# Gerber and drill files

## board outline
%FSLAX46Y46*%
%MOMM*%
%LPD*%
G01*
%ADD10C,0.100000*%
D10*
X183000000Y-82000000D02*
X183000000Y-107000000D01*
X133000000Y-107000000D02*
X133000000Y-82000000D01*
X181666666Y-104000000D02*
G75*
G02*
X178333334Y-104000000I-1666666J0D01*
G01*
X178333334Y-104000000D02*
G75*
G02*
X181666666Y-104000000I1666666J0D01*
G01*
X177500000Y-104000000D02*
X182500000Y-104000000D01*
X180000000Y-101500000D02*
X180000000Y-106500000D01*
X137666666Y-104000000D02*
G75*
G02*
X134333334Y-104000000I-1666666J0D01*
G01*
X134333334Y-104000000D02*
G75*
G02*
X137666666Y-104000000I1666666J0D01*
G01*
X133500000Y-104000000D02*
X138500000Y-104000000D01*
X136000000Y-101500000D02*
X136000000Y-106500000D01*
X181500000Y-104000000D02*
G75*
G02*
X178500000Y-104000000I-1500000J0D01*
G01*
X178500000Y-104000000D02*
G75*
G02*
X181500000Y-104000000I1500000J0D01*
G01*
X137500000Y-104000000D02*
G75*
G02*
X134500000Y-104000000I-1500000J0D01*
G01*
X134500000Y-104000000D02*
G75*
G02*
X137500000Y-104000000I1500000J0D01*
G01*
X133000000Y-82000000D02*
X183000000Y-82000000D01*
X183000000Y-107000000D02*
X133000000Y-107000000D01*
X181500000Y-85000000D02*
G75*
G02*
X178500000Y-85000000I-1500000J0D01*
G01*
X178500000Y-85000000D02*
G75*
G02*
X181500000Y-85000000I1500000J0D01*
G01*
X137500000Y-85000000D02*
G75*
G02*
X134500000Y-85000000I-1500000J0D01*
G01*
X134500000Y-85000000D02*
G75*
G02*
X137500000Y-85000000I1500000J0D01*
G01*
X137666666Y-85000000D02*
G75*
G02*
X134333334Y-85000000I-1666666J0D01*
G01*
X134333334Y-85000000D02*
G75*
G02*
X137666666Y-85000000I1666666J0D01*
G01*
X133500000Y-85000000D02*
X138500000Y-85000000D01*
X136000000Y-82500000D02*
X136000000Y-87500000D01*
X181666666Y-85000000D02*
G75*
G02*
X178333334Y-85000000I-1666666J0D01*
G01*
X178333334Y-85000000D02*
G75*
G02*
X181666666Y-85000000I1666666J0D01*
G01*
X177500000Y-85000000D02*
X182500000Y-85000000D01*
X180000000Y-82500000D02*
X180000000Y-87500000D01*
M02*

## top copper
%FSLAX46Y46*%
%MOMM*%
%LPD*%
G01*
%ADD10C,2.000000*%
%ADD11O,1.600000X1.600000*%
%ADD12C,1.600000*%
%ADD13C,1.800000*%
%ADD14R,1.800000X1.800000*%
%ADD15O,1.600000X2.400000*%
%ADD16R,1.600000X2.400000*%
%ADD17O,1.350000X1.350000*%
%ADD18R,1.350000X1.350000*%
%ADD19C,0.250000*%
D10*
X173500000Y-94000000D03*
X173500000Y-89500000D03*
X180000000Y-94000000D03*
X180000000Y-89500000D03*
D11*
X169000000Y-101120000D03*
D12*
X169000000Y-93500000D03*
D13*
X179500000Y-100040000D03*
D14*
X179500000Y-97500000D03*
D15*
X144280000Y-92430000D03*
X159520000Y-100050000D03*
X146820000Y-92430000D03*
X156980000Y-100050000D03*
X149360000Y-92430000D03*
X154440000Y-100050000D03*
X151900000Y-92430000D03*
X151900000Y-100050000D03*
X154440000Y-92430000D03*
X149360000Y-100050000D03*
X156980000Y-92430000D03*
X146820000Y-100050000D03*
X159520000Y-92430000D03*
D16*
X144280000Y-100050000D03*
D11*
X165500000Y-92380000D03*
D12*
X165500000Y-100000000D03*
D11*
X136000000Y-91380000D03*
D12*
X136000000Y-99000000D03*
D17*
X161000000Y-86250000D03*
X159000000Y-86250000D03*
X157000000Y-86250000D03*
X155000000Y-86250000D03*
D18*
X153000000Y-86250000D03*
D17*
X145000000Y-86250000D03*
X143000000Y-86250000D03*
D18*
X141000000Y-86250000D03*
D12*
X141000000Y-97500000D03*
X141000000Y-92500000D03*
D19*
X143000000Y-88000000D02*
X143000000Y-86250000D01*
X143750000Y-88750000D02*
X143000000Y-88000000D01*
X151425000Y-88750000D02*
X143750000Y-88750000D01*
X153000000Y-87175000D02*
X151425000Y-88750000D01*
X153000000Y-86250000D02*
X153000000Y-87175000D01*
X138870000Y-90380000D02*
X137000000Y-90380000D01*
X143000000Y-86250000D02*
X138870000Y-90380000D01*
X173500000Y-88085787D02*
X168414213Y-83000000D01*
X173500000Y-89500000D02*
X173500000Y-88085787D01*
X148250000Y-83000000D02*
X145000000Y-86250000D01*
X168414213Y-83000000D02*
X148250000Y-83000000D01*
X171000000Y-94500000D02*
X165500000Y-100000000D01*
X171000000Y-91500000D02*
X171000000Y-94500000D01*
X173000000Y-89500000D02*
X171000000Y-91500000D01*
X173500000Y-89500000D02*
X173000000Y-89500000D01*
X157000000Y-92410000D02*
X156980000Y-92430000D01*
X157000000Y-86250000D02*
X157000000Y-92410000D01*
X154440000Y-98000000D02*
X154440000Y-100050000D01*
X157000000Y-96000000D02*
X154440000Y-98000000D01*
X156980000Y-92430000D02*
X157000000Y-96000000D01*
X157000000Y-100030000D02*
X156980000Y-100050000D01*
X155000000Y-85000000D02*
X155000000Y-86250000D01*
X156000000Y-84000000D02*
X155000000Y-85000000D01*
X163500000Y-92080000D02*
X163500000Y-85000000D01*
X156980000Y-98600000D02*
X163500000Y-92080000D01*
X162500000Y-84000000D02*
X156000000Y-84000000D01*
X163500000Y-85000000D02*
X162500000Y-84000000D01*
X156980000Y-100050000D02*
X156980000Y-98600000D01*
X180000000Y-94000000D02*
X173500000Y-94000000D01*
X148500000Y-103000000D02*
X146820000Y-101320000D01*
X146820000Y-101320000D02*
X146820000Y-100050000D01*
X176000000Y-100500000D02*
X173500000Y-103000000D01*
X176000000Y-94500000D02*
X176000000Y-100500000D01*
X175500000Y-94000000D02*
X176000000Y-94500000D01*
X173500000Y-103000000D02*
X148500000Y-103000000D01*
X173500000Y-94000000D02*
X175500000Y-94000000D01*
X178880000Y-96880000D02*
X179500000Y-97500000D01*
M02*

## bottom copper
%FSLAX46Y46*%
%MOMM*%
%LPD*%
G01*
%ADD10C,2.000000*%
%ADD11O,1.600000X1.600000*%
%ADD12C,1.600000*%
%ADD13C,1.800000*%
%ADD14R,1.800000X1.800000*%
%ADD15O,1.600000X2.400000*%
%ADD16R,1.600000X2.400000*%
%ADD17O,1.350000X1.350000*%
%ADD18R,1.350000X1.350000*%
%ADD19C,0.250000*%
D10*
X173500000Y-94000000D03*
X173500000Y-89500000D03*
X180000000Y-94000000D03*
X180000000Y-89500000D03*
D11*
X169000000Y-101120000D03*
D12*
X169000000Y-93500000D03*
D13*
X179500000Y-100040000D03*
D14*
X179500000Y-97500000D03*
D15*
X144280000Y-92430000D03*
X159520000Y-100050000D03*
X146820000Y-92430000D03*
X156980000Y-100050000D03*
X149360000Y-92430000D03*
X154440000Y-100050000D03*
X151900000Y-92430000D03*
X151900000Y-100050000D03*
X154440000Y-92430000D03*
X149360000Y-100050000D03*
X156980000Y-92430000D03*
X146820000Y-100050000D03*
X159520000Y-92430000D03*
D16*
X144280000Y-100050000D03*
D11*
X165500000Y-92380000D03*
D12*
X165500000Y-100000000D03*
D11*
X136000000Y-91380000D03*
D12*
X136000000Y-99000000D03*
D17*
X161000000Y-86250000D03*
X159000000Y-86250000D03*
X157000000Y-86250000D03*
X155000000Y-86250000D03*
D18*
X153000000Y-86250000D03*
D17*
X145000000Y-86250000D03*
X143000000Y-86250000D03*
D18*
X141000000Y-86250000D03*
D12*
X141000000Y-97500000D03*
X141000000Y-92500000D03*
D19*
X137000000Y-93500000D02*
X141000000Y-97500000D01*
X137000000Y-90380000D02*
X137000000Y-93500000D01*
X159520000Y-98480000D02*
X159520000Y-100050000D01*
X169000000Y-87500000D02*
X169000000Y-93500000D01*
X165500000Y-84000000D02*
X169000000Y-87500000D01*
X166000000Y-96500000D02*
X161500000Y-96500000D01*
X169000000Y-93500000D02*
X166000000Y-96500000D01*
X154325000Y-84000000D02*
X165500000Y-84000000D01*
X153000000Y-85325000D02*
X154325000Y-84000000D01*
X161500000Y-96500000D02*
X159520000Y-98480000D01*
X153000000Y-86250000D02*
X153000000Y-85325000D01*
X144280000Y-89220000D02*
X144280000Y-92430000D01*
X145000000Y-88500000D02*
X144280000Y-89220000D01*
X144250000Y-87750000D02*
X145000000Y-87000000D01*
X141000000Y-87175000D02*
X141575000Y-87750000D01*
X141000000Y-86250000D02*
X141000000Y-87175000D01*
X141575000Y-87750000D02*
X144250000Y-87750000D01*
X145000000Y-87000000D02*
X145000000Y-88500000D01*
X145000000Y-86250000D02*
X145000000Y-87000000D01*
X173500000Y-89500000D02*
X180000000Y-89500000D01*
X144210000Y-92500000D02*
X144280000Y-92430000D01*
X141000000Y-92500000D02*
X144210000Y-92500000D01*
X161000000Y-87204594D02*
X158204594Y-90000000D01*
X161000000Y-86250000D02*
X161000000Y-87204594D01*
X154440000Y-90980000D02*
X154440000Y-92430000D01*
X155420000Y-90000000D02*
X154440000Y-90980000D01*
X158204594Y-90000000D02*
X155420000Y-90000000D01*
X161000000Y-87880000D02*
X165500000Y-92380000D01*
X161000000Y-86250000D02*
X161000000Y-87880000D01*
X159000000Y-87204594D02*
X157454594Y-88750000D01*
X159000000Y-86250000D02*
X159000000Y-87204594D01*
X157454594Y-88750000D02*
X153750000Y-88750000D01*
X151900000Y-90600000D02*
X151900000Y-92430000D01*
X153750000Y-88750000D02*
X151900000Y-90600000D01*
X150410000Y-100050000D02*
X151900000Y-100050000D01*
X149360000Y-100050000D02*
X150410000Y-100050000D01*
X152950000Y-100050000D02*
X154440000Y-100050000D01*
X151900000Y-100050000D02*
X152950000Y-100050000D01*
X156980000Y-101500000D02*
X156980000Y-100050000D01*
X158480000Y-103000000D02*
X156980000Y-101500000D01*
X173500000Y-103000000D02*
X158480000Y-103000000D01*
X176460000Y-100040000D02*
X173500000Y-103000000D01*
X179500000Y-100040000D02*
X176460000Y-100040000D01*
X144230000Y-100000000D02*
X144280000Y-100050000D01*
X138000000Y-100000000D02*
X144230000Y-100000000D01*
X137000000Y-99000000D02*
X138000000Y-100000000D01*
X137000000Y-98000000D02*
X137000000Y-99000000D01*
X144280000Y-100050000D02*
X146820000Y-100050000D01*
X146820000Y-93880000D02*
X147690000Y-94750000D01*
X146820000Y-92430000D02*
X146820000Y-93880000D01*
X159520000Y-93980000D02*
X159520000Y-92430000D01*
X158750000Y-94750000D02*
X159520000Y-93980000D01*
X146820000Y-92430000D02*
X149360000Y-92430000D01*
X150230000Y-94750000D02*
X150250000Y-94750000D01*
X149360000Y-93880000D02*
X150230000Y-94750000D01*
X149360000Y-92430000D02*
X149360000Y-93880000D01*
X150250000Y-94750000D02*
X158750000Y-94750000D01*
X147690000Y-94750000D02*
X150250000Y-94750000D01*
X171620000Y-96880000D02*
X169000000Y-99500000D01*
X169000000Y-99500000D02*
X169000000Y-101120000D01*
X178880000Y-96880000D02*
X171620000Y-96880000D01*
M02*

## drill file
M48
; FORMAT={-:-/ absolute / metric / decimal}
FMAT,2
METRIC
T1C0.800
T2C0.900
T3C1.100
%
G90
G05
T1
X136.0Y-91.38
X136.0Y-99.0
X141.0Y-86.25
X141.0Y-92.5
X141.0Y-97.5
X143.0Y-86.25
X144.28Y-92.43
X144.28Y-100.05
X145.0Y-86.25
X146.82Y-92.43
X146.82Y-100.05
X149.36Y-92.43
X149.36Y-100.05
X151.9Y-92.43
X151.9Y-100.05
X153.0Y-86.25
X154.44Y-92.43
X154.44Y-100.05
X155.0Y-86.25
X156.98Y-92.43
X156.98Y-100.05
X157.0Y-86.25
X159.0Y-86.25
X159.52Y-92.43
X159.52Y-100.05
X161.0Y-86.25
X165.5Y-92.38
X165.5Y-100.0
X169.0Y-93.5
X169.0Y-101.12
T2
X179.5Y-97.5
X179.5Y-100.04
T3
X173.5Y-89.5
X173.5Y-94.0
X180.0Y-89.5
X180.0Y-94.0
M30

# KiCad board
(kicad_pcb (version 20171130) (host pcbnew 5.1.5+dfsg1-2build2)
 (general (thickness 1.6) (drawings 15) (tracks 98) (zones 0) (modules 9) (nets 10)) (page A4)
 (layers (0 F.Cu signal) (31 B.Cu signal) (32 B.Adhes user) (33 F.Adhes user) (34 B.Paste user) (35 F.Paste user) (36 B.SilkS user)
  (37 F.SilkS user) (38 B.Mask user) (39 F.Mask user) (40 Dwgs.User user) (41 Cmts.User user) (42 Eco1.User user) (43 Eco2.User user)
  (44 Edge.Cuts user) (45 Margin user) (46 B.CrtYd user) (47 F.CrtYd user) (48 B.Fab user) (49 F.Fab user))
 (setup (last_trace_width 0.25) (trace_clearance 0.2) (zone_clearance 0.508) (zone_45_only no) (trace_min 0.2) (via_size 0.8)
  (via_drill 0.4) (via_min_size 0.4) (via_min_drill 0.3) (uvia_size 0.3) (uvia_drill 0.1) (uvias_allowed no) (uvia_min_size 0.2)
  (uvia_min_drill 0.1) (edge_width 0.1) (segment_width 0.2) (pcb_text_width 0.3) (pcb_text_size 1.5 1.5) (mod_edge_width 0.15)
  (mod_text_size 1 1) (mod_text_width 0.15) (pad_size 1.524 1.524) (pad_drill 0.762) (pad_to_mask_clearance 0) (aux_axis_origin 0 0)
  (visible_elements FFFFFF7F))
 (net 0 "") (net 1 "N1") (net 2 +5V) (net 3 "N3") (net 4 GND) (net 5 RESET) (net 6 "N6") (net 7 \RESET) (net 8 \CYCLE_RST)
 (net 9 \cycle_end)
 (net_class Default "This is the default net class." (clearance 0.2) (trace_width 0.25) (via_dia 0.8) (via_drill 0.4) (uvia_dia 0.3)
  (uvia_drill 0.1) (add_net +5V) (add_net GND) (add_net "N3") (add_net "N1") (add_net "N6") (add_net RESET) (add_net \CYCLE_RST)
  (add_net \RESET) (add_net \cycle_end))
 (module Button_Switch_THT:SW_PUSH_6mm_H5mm (layer F.Cu) (at 180 94 180)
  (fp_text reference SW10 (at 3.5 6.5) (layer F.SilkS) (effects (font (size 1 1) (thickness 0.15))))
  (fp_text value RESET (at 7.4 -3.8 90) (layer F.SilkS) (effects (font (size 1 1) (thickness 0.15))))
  (pad 1 thru_hole circle (at 6.5 0 270) (size 2 2) (drill 1.1) (layers *.Cu *.Mask) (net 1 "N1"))
  (pad 2 thru_hole circle (at 6.5 4.5 270) (size 2 2) (drill 1.1) (layers *.Cu *.Mask) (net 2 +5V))
  (pad 1 thru_hole circle (at 0 0 270) (size 2 2) (drill 1.1) (layers *.Cu *.Mask) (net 1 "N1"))
  (pad 2 thru_hole circle (at 0 4.5 270) (size 2 2) (drill 1.1) (layers *.Cu *.Mask) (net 2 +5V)))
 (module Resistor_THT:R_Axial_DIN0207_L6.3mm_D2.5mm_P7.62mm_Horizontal (layer F.Cu) (at 169 93.5 270)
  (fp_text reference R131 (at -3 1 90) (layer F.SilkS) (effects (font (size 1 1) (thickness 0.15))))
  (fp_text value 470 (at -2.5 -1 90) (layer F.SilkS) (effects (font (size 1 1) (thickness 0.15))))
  (pad 2 thru_hole oval (at 7.62 0 270) (size 1.6 1.6) (drill 0.8) (layers *.Cu *.Mask) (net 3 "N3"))
  (pad 1 thru_hole circle (at 0 0 270) (size 1.6 1.6) (drill 0.8) (layers *.Cu *.Mask) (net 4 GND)))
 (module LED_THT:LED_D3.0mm (layer F.Cu) (at 179.5 97.5 270)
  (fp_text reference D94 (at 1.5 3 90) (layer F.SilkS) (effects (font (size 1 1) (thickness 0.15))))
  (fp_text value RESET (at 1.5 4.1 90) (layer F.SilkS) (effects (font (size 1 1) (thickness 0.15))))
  (pad 2 thru_hole circle (at 2.54 0 270) (size 1.8 1.8) (drill 0.9) (layers *.Cu *.Mask) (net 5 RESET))
  (pad 1 thru_hole rect (at 0 0 270) (size 1.8 1.8) (drill 0.9) (layers *.Cu *.Mask) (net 3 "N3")))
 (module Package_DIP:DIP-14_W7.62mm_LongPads (layer F.Cu) (at 144.28 100.05 90)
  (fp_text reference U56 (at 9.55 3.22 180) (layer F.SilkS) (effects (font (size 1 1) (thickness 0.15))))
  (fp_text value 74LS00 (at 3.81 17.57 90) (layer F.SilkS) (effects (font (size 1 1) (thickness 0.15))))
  (pad 14 thru_hole oval (at 7.62 0 90) (size 2.4 1.6) (drill 0.8) (layers *.Cu *.Mask) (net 2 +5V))
  (pad 7 thru_hole oval (at 0 15.24 90) (size 2.4 1.6) (drill 0.8) (layers *.Cu *.Mask) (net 4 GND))
  (pad 13 thru_hole oval (at 7.62 2.54 90) (size 2.4 1.6) (drill 0.8) (layers *.Cu *.Mask) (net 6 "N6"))
  (pad 6 thru_hole oval (at 0 12.7 90) (size 2.4 1.6) (drill 0.8) (layers *.Cu *.Mask) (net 5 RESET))
  (pad 12 thru_hole oval (at 7.62 5.08 90) (size 2.4 1.6) (drill 0.8) (layers *.Cu *.Mask) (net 6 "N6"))
  (pad 5 thru_hole oval (at 0 10.16 90) (size 2.4 1.6) (drill 0.8) (layers *.Cu *.Mask) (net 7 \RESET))
  (pad 11 thru_hole oval (at 7.62 7.62 90) (size 2.4 1.6) (drill 0.8) (layers *.Cu *.Mask) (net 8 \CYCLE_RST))
  (pad 4 thru_hole oval (at 0 7.62 90) (size 2.4 1.6) (drill 0.8) (layers *.Cu *.Mask) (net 7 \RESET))
  (pad 10 thru_hole oval (at 7.62 10.16 90) (size 2.4 1.6) (drill 0.8) (layers *.Cu *.Mask) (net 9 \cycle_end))
  (pad 3 thru_hole oval (at 0 5.08 90) (size 2.4 1.6) (drill 0.8) (layers *.Cu *.Mask) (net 7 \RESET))
  (pad 9 thru_hole oval (at 7.62 12.7 90) (size 2.4 1.6) (drill 0.8) (layers *.Cu *.Mask) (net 7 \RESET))
  (pad 2 thru_hole oval (at 0 2.54 90) (size 2.4 1.6) (drill 0.8) (layers *.Cu *.Mask) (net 1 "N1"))
  (pad 8 thru_hole oval (at 7.62 15.24 90) (size 2.4 1.6) (drill 0.8) (layers *.Cu *.Mask) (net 6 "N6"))
  (pad 1 thru_hole rect (at 0 0 90) (size 2.4 1.6) (drill 0.8) (layers *.Cu *.Mask) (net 1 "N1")))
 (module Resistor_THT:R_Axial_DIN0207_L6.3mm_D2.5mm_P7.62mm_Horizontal (layer F.Cu) (at 165.5 100 90)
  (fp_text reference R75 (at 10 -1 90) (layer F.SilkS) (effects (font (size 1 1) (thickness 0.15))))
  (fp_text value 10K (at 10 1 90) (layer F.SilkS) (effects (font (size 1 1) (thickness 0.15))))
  (pad 2 thru_hole oval (at 7.62 0 90) (size 1.6 1.6) (drill 0.8) (layers *.Cu *.Mask) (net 9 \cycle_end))
  (pad 1 thru_hole circle (at 0 0 90) (size 1.6 1.6) (drill 0.8) (layers *.Cu *.Mask) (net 2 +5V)))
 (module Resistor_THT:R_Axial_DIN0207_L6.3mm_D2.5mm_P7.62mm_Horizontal (layer F.Cu) (at 136 99 90)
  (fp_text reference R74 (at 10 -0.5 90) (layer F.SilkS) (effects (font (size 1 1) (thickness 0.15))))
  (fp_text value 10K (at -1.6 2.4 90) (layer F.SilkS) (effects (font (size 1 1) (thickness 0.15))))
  (pad 2 thru_hole oval (at 7.62 0 90) (size 1.6 1.6) (drill 0.8) (layers *.Cu *.Mask) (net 4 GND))
  (pad 1 thru_hole circle (at 0 0 90) (size 1.6 1.6) (drill 0.8) (layers *.Cu *.Mask) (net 1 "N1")))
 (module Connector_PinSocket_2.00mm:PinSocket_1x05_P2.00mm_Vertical (layer F.Cu) (at 153 86.25 90)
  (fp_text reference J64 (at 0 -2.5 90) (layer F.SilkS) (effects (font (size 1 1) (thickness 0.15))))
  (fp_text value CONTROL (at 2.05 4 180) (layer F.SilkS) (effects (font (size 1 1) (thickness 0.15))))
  (pad 5 thru_hole oval (at 0 8 90) (size 1.35 1.35) (drill 0.8) (layers *.Cu *.Mask) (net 9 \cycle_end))
  (pad 4 thru_hole oval (at 0 6 90) (size 1.35 1.35) (drill 0.8) (layers *.Cu *.Mask) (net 8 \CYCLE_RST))
  (pad 3 thru_hole oval (at 0 4 90) (size 1.35 1.35) (drill 0.8) (layers *.Cu *.Mask) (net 7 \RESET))
  (pad 2 thru_hole oval (at 0 2 90) (size 1.35 1.35) (drill 0.8) (layers *.Cu *.Mask) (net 5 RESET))
  (pad 1 thru_hole rect (at 0 0 90) (size 1.35 1.35) (drill 0.8) (layers *.Cu *.Mask) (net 4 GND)))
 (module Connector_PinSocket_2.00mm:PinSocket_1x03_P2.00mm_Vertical (layer F.Cu) (at 141 86.25 90)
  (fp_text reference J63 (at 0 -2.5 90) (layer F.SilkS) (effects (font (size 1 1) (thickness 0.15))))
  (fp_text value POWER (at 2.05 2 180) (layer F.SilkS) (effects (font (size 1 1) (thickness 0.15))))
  (pad 3 thru_hole oval (at 0 4 90) (size 1.35 1.35) (drill 0.8) (layers *.Cu *.Mask) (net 2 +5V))
  (pad 2 thru_hole oval (at 0 2 90) (size 1.35 1.35) (drill 0.8) (layers *.Cu *.Mask) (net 4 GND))
  (pad 1 thru_hole rect (at 0 0 90) (size 1.35 1.35) (drill 0.8) (layers *.Cu *.Mask) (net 2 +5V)))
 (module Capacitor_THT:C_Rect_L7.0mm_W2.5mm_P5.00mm (layer F.Cu) (at 141 92.5 270)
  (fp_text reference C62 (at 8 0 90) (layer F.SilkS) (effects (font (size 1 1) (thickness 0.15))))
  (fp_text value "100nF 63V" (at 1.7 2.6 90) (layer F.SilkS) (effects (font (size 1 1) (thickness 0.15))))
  (pad 2 thru_hole circle (at 5 0 270) (size 1.6 1.6) (drill 0.8) (layers *.Cu *.Mask) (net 4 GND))
  (pad 1 thru_hole circle (at 0 0 270) (size 1.6 1.6) (drill 0.8) (layers *.Cu *.Mask) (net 2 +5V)))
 (gr_line (start 183 82) (end 183 107) (layer Edge.Cuts) (width 0.1))
 (gr_line (start 133 107) (end 133 82) (layer Edge.Cuts) (width 0.1))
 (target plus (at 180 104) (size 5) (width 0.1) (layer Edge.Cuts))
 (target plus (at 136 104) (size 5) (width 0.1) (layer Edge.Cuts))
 (gr_circle (center 180 104) (end 181.5 104) (layer Edge.Cuts) (width 0.1))
 (gr_circle (center 136 104) (end 137.5 104) (layer Edge.Cuts) (width 0.1))
 (gr_line (start 133 82) (end 183 82) (layer Edge.Cuts) (width 0.1))
 (gr_line (start 183 107) (end 133 107) (layer Edge.Cuts) (width 0.1))
 (gr_circle (center 180 85) (end 181.5 85) (layer Edge.Cuts) (width 0.1))
 (gr_circle (center 136 85) (end 137.5 85) (layer Edge.Cuts) (width 0.1))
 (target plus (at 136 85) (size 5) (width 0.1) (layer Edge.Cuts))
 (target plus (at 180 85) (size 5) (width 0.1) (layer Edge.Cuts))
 (segment (start 143 88) (end 143 86.25) (width 0.25) (layer F.Cu) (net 4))
 (segment (start 143.75 88.75) (end 143 88) (width 0.25) (layer F.Cu) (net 4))
 (segment (start 151.425 88.75) (end 143.75 88.75) (width 0.25) (layer F.Cu) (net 4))
 (segment (start 153 87.175) (end 151.425 88.75) (width 0.25) (layer F.Cu) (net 4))
 (segment (start 153 86.25) (end 153 87.175) (width 0.25) (layer F.Cu) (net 4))
 (segment (start 138.87 90.38) (end 137 90.38) (width 0.25) (layer F.Cu) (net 4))
 (segment (start 143 86.25) (end 138.87 90.38) (width 0.25) (layer F.Cu) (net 4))
 (segment (start 137 93.5) (end 141 97.5) (width 0.25) (layer B.Cu) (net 4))
 (segment (start 137 90.38) (end 137 93.5) (width 0.25) (layer B.Cu) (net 4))
 (segment (start 159.52 98.48) (end 159.52 100.05) (width 0.25) (layer B.Cu) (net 4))
 (segment (start 169 87.5) (end 169 93.5) (width 0.25) (layer B.Cu) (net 4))
 (segment (start 165.5 84) (end 169 87.5) (width 0.25) (layer B.Cu) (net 4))
 (segment (start 166 96.5) (end 161.5 96.5) (width 0.25) (layer B.Cu) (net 4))
 (segment (start 169 93.5) (end 166 96.5) (width 0.25) (layer B.Cu) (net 4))
 (segment (start 154.325 84) (end 165.5 84) (width 0.25) (layer B.Cu) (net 4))
 (segment (start 153 85.325) (end 154.325 84) (width 0.25) (layer B.Cu) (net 4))
 (segment (start 161.5 96.5) (end 159.52 98.48) (width 0.25) (layer B.Cu) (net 4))
 (segment (start 153 86.25) (end 153 85.325) (width 0.25) (layer B.Cu) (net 4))
 (segment (start 144.28 89.22) (end 144.28 92.43) (width 0.25) (layer B.Cu) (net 2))
 (segment (start 145 88.5) (end 144.28 89.22) (width 0.25) (layer B.Cu) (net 2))
 (segment (start 144.25 87.75) (end 145 87) (width 0.25) (layer B.Cu) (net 2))
 (segment (start 141 87.175) (end 141.575 87.75) (width 0.25) (layer B.Cu) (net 2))
 (segment (start 141 86.25) (end 141 87.175) (width 0.25) (layer B.Cu) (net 2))
 (segment (start 141.575 87.75) (end 144.25 87.75) (width 0.25) (layer B.Cu) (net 2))
 (segment (start 145 87) (end 145 88.5) (width 0.25) (layer B.Cu) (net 2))
 (segment (start 145 86.25) (end 145 87) (width 0.25) (layer B.Cu) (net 2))
 (segment (start 173.5 89.5) (end 180 89.5) (width 0.25) (layer B.Cu) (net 2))
 (segment (start 173.5 88.085787) (end 168.414213 83) (width 0.25) (layer F.Cu) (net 2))
 (segment (start 173.5 89.5) (end 173.5 88.085787) (width 0.25) (layer F.Cu) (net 2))
 (segment (start 148.25 83) (end 145 86.25) (width 0.25) (layer F.Cu) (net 2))
 (segment (start 168.414213 83) (end 148.25 83) (width 0.25) (layer F.Cu) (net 2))
 (segment (start 171 94.5) (end 165.5 100) (width 0.25) (layer F.Cu) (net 2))
 (segment (start 171 91.5) (end 171 94.5) (width 0.25) (layer F.Cu) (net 2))
 (segment (start 173 89.5) (end 171 91.5) (width 0.25) (layer F.Cu) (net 2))
 (segment (start 173.5 89.5) (end 173 89.5) (width 0.25) (layer F.Cu) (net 2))
 (segment (start 144.21 92.5) (end 144.28 92.43) (width 0.25) (layer B.Cu) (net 2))
 (segment (start 141 92.5) (end 144.21 92.5) (width 0.25) (layer B.Cu) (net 2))
 (segment (start 161 87.204594) (end 158.204594 90) (width 0.25) (layer B.Cu) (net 9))
 (segment (start 161 86.25) (end 161 87.204594) (width 0.25) (layer B.Cu) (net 9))
 (segment (start 154.44 90.98) (end 154.44 92.43) (width 0.25) (layer B.Cu) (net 9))
 (segment (start 155.42 90) (end 154.44 90.98) (width 0.25) (layer B.Cu) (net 9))
 (segment (start 158.204594 90) (end 155.42 90) (width 0.25) (layer B.Cu) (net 9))
 (segment (start 161 87.88) (end 165.5 92.38) (width 0.25) (layer B.Cu) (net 9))
 (segment (start 161 86.25) (end 161 87.88) (width 0.25) (layer B.Cu) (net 9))
 (segment (start 159 87.204594) (end 157.454594 88.75) (width 0.25) (layer B.Cu) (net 8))
 (segment (start 159 86.25) (end 159 87.204594) (width 0.25) (layer B.Cu) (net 8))
 (segment (start 157.454594 88.75) (end 153.75 88.75) (width 0.25) (layer B.Cu) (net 8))
 (segment (start 151.9 90.6) (end 151.9 92.43) (width 0.25) (layer B.Cu) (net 8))
 (segment (start 153.75 88.75) (end 151.9 90.6) (width 0.25) (layer B.Cu) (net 8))
 (segment (start 150.41 100.05) (end 151.9 100.05) (width 0.25) (layer B.Cu) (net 7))
 (segment (start 149.36 100.05) (end 150.41 100.05) (width 0.25) (layer B.Cu) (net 7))
 (segment (start 152.95 100.05) (end 154.44 100.05) (width 0.25) (layer B.Cu) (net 7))
 (segment (start 151.9 100.05) (end 152.95 100.05) (width 0.25) (layer B.Cu) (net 7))
 (segment (start 157 92.41) (end 156.98 92.43) (width 0.25) (layer F.Cu) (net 7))
 (segment (start 157 86.25) (end 157 92.41) (width 0.25) (layer F.Cu) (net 7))
 (segment (start 154.44 98) (end 154.44 100.05) (width 0.25) (layer F.Cu) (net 7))
 (segment (start 157 96) (end 154.44 98) (width 0.25) (layer F.Cu) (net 7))
 (segment (start 156.98 92.43) (end 157 96) (width 0.25) (layer F.Cu) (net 7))
 (segment (start 157 100.03) (end 156.98 100.05) (width 0.25) (layer F.Cu) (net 5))
 (segment (start 155 85) (end 155 86.25) (width 0.25) (layer F.Cu) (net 5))
 (segment (start 156 84) (end 155 85) (width 0.25) (layer F.Cu) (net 5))
 (segment (start 163.5 92.08) (end 163.5 85) (width 0.25) (layer F.Cu) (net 5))
 (segment (start 156.98 98.6) (end 163.5 92.08) (width 0.25) (layer F.Cu) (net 5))
 (segment (start 162.5 84) (end 156 84) (width 0.25) (layer F.Cu) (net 5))
 (segment (start 163.5 85) (end 162.5 84) (width 0.25) (layer F.Cu) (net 5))
 (segment (start 156.98 100.05) (end 156.98 98.6) (width 0.25) (layer F.Cu) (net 5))
 (segment (start 156.98 101.5) (end 156.98 100.05) (width 0.25) (layer B.Cu) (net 5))
 (segment (start 158.48 103) (end 156.98 101.5) (width 0.25) (layer B.Cu) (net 5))
 (segment (start 173.5 103) (end 158.48 103) (width 0.25) (layer B.Cu) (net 5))
 (segment (start 176.46 100.04) (end 173.5 103) (width 0.25) (layer B.Cu) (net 5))
 (segment (start 179.5 100.04) (end 176.46 100.04) (width 0.25) (layer B.Cu) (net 5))
 (segment (start 180 94) (end 173.5 94) (width 0.25) (layer F.Cu) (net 1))
 (segment (start 144.23 100) (end 144.28 100.05) (width 0.25) (layer B.Cu) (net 1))
 (segment (start 138 100) (end 144.23 100) (width 0.25) (layer B.Cu) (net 1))
 (segment (start 137 99) (end 138 100) (width 0.25) (layer B.Cu) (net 1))
 (segment (start 137 98) (end 137 99) (width 0.25) (layer B.Cu) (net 1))
 (segment (start 144.28 100.05) (end 146.82 100.05) (width 0.25) (layer B.Cu) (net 1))
 (segment (start 148.5 103) (end 146.82 101.32) (width 0.25) (layer F.Cu) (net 1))
 (segment (start 146.82 101.32) (end 146.82 100.05) (width 0.25) (layer F.Cu) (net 1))
 (segment (start 176 100.5) (end 173.5 103) (width 0.25) (layer F.Cu) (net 1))
 (segment (start 176 94.5) (end 176 100.5) (width 0.25) (layer F.Cu) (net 1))
 (segment (start 175.5 94) (end 176 94.5) (width 0.25) (layer F.Cu) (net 1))
 (segment (start 173.5 103) (end 148.5 103) (width 0.25) (layer F.Cu) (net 1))
 (segment (start 173.5 94) (end 175.5 94) (width 0.25) (layer F.Cu) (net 1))
 (segment (start 146.82 93.88) (end 147.69 94.75) (width 0.25) (layer B.Cu) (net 6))
 (segment (start 146.82 92.43) (end 146.82 93.88) (width 0.25) (layer B.Cu) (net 6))
 (segment (start 159.52 93.98) (end 159.52 92.43) (width 0.25) (layer B.Cu) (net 6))
 (segment (start 158.75 94.75) (end 159.52 93.98) (width 0.25) (layer B.Cu) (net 6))
 (segment (start 146.82 92.43) (end 149.36 92.43) (width 0.25) (layer B.Cu) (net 6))
 (segment (start 150.23 94.75) (end 150.25 94.75) (width 0.25) (layer B.Cu) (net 6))
 (segment (start 149.36 93.88) (end 150.23 94.75) (width 0.25) (layer B.Cu) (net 6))
 (segment (start 149.36 92.43) (end 149.36 93.88) (width 0.25) (layer B.Cu) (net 6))
 (segment (start 150.25 94.75) (end 158.75 94.75) (width 0.25) (layer B.Cu) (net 6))
 (segment (start 147.69 94.75) (end 150.25 94.75) (width 0.25) (layer B.Cu) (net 6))
 (segment (start 178.88 96.88) (end 179.5 97.5) (width 0.25) (layer F.Cu) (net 3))
 (segment (start 171.62 96.88) (end 169 99.5) (width 0.25) (layer B.Cu) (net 3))
 (segment (start 169 99.5) (end 169 101.12) (width 0.25) (layer B.Cu) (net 3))
 (segment (start 178.88 96.88) (end 171.62 96.88) (width 0.25) (layer B.Cu) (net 3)))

